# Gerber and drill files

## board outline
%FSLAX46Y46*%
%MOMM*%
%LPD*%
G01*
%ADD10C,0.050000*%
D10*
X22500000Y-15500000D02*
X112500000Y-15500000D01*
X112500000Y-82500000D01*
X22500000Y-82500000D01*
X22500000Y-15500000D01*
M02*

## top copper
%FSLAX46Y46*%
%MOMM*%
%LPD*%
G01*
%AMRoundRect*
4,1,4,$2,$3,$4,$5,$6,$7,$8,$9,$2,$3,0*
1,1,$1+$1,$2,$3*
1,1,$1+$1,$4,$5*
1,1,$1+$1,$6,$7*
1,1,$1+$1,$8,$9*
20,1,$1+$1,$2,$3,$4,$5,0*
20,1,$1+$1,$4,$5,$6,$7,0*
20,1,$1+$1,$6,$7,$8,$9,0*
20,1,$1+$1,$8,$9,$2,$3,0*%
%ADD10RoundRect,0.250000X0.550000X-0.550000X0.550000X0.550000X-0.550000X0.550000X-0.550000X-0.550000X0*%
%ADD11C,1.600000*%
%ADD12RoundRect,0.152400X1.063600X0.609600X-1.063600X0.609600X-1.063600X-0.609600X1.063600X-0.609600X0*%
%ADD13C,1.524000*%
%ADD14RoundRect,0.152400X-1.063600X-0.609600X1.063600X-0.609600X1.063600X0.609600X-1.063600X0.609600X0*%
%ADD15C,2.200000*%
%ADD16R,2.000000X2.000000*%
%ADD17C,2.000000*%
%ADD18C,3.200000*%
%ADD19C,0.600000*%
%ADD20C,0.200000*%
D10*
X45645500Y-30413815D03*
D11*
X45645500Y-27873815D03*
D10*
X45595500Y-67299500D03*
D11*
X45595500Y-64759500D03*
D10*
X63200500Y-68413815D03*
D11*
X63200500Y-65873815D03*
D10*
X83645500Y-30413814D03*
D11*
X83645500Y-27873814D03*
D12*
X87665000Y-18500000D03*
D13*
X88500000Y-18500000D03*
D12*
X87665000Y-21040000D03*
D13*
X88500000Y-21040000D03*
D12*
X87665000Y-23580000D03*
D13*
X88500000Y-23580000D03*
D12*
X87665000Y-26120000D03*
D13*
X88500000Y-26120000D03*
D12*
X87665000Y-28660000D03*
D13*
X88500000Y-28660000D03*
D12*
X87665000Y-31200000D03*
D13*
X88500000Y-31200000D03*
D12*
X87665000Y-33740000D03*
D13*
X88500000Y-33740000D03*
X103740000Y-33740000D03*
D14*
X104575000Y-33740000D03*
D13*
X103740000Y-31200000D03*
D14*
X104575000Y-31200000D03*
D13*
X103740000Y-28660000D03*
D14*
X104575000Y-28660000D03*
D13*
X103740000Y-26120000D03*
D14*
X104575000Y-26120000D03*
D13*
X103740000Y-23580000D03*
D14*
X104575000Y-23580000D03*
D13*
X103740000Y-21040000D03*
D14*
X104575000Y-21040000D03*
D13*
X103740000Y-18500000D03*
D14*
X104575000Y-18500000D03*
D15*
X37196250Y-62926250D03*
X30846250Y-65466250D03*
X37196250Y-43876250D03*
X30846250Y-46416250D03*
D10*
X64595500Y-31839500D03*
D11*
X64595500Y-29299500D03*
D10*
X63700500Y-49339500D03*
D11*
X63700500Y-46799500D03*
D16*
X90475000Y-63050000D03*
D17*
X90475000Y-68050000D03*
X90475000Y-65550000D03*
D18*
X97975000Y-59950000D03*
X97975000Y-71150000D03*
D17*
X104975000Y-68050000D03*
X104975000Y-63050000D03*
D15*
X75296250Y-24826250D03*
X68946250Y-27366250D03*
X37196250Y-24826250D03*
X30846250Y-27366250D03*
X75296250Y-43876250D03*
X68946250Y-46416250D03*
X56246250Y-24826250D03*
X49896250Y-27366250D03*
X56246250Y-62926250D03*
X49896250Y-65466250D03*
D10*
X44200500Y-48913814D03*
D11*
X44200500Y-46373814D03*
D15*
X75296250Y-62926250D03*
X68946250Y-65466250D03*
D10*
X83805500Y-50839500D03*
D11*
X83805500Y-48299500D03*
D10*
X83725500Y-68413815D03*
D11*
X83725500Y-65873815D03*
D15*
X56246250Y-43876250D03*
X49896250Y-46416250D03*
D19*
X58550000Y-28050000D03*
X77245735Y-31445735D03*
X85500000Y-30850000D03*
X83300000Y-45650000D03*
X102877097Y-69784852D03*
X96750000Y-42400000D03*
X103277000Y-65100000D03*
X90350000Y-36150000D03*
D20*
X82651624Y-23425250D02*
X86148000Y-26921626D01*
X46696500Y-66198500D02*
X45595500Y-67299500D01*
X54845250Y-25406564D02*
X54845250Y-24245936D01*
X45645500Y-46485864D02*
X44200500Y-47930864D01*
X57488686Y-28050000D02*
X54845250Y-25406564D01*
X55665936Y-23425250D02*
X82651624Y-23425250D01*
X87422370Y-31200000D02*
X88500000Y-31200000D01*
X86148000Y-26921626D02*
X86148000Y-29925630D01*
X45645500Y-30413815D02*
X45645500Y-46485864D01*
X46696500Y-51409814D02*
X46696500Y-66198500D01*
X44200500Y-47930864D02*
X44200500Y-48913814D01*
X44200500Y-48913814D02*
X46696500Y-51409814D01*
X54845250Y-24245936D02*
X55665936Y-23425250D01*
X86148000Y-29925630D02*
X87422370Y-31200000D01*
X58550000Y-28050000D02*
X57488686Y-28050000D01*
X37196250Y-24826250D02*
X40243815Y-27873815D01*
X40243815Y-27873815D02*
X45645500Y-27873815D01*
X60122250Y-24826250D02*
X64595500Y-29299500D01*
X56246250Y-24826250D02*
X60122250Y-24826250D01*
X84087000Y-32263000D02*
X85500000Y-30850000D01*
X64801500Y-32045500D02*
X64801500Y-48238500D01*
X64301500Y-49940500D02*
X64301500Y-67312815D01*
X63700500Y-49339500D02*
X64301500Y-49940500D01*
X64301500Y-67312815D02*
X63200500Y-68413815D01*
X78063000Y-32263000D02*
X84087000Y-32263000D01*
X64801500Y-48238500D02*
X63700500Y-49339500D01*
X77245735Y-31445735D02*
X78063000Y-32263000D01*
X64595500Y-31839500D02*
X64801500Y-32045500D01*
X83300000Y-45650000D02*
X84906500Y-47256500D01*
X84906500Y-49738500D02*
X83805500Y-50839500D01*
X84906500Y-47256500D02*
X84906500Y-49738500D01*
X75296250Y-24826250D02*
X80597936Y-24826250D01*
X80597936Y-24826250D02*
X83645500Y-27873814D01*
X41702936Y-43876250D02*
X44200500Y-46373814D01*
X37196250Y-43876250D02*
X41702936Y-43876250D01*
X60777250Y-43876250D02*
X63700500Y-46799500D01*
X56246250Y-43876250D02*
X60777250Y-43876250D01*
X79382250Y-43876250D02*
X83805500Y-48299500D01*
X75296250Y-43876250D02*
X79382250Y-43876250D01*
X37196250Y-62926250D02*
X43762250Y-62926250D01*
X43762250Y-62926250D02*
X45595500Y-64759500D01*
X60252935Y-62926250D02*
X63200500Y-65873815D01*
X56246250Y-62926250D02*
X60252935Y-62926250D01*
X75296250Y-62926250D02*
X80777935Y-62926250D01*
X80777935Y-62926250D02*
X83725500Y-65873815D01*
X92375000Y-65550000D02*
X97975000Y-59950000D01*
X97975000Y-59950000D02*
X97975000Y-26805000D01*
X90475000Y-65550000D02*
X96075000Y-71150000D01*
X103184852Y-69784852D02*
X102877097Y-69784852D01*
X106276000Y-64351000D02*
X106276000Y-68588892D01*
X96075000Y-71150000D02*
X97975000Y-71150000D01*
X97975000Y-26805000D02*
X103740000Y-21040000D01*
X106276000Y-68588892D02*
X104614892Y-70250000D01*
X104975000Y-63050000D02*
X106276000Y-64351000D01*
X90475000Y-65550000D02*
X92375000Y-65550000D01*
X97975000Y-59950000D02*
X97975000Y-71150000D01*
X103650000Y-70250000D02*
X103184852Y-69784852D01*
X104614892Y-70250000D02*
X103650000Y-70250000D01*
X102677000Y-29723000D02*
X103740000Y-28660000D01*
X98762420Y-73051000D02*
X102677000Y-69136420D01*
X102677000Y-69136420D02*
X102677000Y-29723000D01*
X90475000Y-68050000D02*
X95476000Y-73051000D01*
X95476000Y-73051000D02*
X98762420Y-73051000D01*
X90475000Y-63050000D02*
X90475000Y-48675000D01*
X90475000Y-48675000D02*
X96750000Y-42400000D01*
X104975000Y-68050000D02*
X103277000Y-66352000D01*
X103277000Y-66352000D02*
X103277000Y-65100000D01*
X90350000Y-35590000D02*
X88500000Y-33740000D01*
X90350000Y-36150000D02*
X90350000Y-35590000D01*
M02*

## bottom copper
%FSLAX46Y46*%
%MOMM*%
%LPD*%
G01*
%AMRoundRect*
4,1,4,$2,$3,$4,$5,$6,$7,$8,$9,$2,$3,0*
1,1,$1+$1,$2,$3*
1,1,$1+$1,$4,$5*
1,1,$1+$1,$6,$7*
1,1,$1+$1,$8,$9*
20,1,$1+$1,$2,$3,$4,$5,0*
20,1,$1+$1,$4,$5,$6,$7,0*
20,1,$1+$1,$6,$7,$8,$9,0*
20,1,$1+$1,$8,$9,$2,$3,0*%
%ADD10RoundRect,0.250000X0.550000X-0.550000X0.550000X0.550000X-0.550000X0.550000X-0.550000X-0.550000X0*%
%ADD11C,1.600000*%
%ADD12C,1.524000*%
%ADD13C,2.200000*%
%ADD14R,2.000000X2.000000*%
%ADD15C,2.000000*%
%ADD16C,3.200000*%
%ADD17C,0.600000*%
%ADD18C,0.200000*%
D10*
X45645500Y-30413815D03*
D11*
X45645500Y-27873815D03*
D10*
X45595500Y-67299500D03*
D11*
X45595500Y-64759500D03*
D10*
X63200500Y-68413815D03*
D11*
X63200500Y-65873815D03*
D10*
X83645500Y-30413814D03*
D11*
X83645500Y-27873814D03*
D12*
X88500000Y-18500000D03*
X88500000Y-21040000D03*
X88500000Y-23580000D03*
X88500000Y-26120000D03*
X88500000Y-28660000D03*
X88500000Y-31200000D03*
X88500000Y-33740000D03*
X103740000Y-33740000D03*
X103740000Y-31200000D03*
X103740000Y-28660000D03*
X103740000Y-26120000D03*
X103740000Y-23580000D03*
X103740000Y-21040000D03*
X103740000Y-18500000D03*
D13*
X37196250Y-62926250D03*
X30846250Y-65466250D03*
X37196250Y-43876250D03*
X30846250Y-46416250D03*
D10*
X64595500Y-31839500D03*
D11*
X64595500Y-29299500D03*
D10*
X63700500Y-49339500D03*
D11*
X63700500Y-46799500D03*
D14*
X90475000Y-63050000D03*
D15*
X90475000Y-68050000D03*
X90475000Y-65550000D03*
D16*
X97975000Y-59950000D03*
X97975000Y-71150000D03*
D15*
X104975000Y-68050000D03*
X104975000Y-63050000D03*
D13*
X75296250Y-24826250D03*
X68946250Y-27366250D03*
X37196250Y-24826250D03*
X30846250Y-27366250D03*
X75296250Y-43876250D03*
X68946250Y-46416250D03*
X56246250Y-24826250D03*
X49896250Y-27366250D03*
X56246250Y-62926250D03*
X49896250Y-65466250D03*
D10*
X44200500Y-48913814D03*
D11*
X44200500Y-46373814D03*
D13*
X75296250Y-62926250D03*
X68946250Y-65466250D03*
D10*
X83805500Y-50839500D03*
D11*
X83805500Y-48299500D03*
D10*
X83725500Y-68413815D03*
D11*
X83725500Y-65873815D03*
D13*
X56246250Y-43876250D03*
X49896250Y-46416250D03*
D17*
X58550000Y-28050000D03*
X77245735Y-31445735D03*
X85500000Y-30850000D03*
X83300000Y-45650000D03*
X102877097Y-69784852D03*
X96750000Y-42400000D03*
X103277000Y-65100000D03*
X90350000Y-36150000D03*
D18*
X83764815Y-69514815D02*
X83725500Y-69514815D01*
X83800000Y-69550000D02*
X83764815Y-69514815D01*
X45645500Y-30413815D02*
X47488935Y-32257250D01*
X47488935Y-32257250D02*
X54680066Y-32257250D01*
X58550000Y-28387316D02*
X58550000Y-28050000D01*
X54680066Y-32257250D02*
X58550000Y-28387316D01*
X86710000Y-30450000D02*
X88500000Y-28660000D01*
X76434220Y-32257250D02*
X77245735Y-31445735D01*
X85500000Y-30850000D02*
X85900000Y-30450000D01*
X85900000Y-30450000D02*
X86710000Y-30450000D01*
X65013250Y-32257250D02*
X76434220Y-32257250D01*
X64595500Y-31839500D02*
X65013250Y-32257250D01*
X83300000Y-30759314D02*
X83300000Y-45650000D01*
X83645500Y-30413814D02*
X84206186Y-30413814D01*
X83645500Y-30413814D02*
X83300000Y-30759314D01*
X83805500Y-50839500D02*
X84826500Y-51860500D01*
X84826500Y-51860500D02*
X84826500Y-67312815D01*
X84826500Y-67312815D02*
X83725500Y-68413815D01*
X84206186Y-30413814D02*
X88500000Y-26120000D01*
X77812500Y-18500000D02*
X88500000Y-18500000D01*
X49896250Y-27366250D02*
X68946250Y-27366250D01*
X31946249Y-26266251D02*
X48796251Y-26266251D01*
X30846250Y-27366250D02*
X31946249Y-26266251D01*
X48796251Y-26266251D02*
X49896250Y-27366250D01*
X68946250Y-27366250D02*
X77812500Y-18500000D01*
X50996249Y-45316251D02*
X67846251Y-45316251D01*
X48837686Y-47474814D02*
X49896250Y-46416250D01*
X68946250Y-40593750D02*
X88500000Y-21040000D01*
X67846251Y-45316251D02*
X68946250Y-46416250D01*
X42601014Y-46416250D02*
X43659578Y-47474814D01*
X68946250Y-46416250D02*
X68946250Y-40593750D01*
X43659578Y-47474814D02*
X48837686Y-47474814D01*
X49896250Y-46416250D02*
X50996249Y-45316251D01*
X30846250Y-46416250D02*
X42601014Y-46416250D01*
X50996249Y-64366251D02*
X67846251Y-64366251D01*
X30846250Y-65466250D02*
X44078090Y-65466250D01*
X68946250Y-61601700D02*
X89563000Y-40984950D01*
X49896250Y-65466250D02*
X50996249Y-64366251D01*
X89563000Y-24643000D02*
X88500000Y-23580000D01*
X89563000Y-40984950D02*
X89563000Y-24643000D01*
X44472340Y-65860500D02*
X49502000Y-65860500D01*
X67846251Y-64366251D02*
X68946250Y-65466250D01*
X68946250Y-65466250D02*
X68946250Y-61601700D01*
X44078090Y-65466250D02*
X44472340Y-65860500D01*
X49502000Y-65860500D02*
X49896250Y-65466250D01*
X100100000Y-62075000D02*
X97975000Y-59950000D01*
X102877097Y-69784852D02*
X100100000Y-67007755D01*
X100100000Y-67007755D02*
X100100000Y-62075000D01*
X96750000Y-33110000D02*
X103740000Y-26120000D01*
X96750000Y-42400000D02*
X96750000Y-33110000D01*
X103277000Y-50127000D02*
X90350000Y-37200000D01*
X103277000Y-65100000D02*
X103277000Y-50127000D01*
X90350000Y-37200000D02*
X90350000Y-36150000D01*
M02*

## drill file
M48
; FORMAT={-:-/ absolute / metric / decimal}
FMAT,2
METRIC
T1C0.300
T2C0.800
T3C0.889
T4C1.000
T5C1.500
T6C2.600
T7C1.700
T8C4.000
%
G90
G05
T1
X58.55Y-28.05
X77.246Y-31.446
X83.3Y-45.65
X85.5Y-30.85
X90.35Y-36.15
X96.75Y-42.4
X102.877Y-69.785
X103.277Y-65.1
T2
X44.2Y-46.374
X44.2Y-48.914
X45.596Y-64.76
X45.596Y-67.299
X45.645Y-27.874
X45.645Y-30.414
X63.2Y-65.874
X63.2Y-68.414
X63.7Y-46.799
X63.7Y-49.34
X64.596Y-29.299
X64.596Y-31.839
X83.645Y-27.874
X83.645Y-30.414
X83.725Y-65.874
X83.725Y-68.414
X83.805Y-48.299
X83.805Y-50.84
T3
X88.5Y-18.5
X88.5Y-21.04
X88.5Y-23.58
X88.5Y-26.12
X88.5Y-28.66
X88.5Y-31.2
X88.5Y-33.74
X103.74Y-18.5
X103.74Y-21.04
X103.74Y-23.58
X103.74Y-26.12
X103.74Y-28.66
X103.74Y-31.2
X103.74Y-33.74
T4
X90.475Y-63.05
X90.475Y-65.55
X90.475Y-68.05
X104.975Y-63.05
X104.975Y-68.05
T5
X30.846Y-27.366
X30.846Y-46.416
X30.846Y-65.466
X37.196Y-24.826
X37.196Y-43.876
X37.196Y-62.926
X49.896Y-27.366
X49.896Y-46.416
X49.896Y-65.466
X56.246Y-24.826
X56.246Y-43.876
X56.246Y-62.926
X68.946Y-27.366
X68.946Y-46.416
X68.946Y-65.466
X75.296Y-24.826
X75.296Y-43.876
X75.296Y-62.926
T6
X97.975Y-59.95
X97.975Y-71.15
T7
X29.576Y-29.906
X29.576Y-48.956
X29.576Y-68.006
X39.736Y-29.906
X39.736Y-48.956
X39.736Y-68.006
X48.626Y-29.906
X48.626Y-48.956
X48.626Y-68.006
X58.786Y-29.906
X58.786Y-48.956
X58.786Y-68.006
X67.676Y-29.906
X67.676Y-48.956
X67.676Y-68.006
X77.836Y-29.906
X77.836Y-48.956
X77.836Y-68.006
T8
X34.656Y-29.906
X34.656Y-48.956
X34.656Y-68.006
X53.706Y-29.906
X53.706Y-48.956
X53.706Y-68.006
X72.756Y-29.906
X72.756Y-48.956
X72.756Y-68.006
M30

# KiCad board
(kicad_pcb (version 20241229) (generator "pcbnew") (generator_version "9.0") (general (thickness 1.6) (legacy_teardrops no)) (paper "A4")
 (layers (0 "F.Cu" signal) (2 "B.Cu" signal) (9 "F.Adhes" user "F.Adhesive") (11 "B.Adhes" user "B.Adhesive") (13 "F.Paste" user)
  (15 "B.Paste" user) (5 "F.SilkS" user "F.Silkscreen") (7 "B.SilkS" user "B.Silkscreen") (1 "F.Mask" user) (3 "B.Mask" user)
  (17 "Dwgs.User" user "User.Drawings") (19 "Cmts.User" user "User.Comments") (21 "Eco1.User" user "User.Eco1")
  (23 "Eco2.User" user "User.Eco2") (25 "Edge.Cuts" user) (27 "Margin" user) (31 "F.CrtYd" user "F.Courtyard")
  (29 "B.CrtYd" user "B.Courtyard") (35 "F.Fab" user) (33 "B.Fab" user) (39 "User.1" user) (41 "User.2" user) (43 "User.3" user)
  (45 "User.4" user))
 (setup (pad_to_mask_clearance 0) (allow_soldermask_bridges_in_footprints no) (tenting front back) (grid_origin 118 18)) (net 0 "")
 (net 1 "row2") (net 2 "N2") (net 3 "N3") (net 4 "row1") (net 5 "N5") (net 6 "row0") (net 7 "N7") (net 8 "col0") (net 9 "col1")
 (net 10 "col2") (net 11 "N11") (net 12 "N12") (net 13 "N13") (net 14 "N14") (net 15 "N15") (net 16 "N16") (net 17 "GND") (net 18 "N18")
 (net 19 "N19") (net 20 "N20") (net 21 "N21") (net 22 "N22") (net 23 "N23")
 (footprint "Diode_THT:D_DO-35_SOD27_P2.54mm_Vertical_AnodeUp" (layer "F.Cu") (at 45.6455 30.413815 90)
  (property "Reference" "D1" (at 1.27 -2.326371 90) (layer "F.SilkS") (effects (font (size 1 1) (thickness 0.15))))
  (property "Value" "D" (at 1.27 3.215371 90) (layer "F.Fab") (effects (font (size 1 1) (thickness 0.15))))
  (pad "1" thru_hole roundrect (at 0 0 90) (size 1.6 1.6) (drill 0.8) (layers "*.Cu" "*.Mask") (remove_unused_layers no)
   (roundrect_rratio 0.15625) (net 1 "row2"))
  (pad "2" thru_hole circle (at 2.54 0 90) (size 1.6 1.6) (drill 0.8) (layers "*.Cu" "*.Mask") (remove_unused_layers no) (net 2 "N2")))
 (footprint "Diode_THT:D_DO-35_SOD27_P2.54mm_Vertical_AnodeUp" (layer "F.Cu") (at 45.5955 67.2995 90)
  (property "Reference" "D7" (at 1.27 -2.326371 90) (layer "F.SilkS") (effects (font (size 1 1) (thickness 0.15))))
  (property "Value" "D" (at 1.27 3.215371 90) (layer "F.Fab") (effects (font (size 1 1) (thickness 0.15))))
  (pad "1" thru_hole roundrect (at 0 0 90) (size 1.6 1.6) (drill 0.8) (layers "*.Cu" "*.Mask") (remove_unused_layers no)
   (roundrect_rratio 0.15625) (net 1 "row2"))
  (pad "2" thru_hole circle (at 2.54 0 90) (size 1.6 1.6) (drill 0.8) (layers "*.Cu" "*.Mask") (remove_unused_layers no) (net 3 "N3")))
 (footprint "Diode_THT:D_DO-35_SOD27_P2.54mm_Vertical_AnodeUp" (layer "F.Cu") (at 63.2005 68.413815 90)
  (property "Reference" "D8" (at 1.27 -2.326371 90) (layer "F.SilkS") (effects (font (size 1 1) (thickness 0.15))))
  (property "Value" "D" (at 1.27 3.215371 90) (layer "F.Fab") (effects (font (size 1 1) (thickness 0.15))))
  (pad "1" thru_hole roundrect (at 0 0 90) (size 1.6 1.6) (drill 0.8) (layers "*.Cu" "*.Mask") (remove_unused_layers no)
   (roundrect_rratio 0.15625) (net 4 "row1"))
  (pad "2" thru_hole circle (at 2.54 0 90) (size 1.6 1.6) (drill 0.8) (layers "*.Cu" "*.Mask") (remove_unused_layers no) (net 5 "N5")))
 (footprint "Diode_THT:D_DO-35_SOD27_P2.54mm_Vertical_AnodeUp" (layer "F.Cu") (at 83.6455 30.413814 90)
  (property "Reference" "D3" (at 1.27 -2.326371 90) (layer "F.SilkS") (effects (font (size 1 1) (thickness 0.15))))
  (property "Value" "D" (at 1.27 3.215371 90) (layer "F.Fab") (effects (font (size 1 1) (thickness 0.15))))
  (pad "1" thru_hole roundrect (at 0 0 90) (size 1.6 1.6) (drill 0.8) (layers "*.Cu" "*.Mask") (remove_unused_layers no)
   (roundrect_rratio 0.15625) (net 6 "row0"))
  (pad "2" thru_hole circle (at 2.54 0 90) (size 1.6 1.6) (drill 0.8) (layers "*.Cu" "*.Mask") (remove_unused_layers no) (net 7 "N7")))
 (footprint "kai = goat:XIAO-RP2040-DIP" (layer "F.Cu") (at 96.12 26.12)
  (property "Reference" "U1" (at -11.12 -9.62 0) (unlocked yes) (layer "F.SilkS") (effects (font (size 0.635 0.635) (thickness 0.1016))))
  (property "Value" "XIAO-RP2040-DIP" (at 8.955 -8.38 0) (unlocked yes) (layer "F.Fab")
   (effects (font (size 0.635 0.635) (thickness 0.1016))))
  (pad "1" smd roundrect (at -8.455 -7.62 180) (size 2.432 1.524) (layers "F.Cu" "F.Mask") (roundrect_rratio 0.1) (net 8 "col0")
   (thermal_bridge_angle 45))
  (pad "1" thru_hole circle (at -7.62 -7.62 180) (size 1.524 1.524) (drill 0.889) (layers "*.Cu" "*.Mask") (remove_unused_layers no)
   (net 8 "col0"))
  (pad "2" smd roundrect (at -8.455 -5.08 180) (size 2.432 1.524) (layers "F.Cu" "F.Mask") (roundrect_rratio 0.1) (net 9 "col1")
   (thermal_bridge_angle 45))
  (pad "2" thru_hole circle (at -7.62 -5.08 180) (size 1.524 1.524) (drill 0.889) (layers "*.Cu" "*.Mask") (remove_unused_layers no)
   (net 9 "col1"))
  (pad "3" smd roundrect (at -8.455 -2.54 180) (size 2.432 1.524) (layers "F.Cu" "F.Mask") (roundrect_rratio 0.1) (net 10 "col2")
   (thermal_bridge_angle 45))
  (pad "3" thru_hole circle (at -7.62 -2.54 180) (size 1.524 1.524) (drill 0.889) (layers "*.Cu" "*.Mask") (remove_unused_layers no)
   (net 10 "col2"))
  (pad "4" smd roundrect (at -8.455 0 180) (size 2.432 1.524) (layers "F.Cu" "F.Mask") (roundrect_rratio 0.1) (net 6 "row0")
   (thermal_bridge_angle 45))
  (pad "4" thru_hole circle (at -7.62 0 180) (size 1.524 1.524) (drill 0.889) (layers "*.Cu" "*.Mask") (remove_unused_layers no)
   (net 6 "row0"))
  (pad "5" smd roundrect (at -8.455 2.54 180) (size 2.432 1.524) (layers "F.Cu" "F.Mask") (roundrect_rratio 0.1) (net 4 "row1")
   (thermal_bridge_angle 45))
  (pad "5" thru_hole circle (at -7.62 2.54 180) (size 1.524 1.524) (drill 0.889) (layers "*.Cu" "*.Mask") (remove_unused_layers no)
   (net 4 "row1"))
  (pad "6" smd roundrect (at -8.455 5.08 180) (size 2.432 1.524) (layers "F.Cu" "F.Mask") (roundrect_rratio 0.1) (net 1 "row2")
   (thermal_bridge_angle 45))
  (pad "6" thru_hole circle (at -7.62 5.08 180) (size 1.524 1.524) (drill 0.889) (layers "*.Cu" "*.Mask") (remove_unused_layers no)
   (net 1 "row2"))
  (pad "7" smd roundrect (at -8.455 7.62 180) (size 2.432 1.524) (layers "F.Cu" "F.Mask") (roundrect_rratio 0.1) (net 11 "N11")
   (thermal_bridge_angle 45))
  (pad "7" thru_hole circle (at -7.62 7.62 180) (size 1.524 1.524) (drill 0.889) (layers "*.Cu" "*.Mask") (remove_unused_layers no)
   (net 11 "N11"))
  (pad "8" thru_hole circle (at 7.62 7.62) (size 1.524 1.524) (drill 0.889) (layers "*.Cu" "*.Mask") (remove_unused_layers no)
   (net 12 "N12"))
  (pad "8" smd roundrect (at 8.455 7.62) (size 2.432 1.524) (layers "F.Cu" "F.Mask") (roundrect_rratio 0.1) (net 12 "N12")
   (thermal_bridge_angle 45))
  (pad "9" thru_hole circle (at 7.62 5.08) (size 1.524 1.524) (drill 0.889) (layers "*.Cu" "*.Mask") (remove_unused_layers no)
   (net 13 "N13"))
  (pad "9" smd roundrect (at 8.455 5.08) (size 2.432 1.524) (layers "F.Cu" "F.Mask") (roundrect_rratio 0.1) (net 13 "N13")
   (thermal_bridge_angle 45))
  (pad "10" thru_hole circle (at 7.62 2.54) (size 1.524 1.524) (drill 0.889) (layers "*.Cu" "*.Mask") (remove_unused_layers no)
   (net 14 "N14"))
  (pad "10" smd roundrect (at 8.455 2.54) (size 2.432 1.524) (layers "F.Cu" "F.Mask") (roundrect_rratio 0.1) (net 14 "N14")
   (thermal_bridge_angle 45))
  (pad "11" thru_hole circle (at 7.62 0) (size 1.524 1.524) (drill 0.889) (layers "*.Cu" "*.Mask") (remove_unused_layers no) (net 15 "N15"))
  (pad "11" smd roundrect (at 8.455 0) (size 2.432 1.524) (layers "F.Cu" "F.Mask") (roundrect_rratio 0.1) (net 15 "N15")
   (thermal_bridge_angle 45))
  (pad "12" thru_hole circle (at 7.62 -2.54) (size 1.524 1.524) (drill 0.889) (layers "*.Cu" "*.Mask") (remove_unused_layers no)
   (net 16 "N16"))
  (pad "12" smd roundrect (at 8.455 -2.54) (size 2.432 1.524) (layers "F.Cu" "F.Mask") (roundrect_rratio 0.1) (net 16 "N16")
   (thermal_bridge_angle 45))
  (pad "13" thru_hole circle (at 7.62 -5.08) (size 1.524 1.524) (drill 0.889) (layers "*.Cu" "*.Mask") (remove_unused_layers no)
   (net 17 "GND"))
  (pad "13" smd roundrect (at 8.455 -5.08) (size 2.432 1.524) (layers "F.Cu" "F.Mask") (roundrect_rratio 0.1) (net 17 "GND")
   (thermal_bridge_angle 45))
  (pad "14" thru_hole circle (at 7.62 -7.62) (size 1.524 1.524) (drill 0.889) (layers "*.Cu" "*.Mask") (remove_unused_layers no)
   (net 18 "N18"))
  (pad "14" smd roundrect (at 8.455 -7.62) (size 2.432 1.524) (layers "F.Cu" "F.Mask") (roundrect_rratio 0.1) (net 18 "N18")
   (thermal_bridge_angle 45)))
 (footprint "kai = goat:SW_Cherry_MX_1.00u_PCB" (layer "F.Cu") (at 37.19625 62.92625)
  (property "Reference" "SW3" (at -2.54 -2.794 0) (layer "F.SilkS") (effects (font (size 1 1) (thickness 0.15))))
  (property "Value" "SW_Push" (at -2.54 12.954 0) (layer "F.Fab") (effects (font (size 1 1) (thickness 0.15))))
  (pad "" np_thru_hole circle (at -7.62 5.08) (size 1.7 1.7) (drill 1.7) (layers "*.Cu" "*.Mask"))
  (pad "" np_thru_hole circle (at -2.54 5.08) (size 4 4) (drill 4) (layers "*.Cu" "*.Mask"))
  (pad "" np_thru_hole circle (at 2.54 5.08) (size 1.7 1.7) (drill 1.7) (layers "*.Cu" "*.Mask"))
  (pad "1" thru_hole circle (at 0 0) (size 2.2 2.2) (drill 1.5) (layers "*.Cu" "*.Mask") (remove_unused_layers no) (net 3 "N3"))
  (pad "2" thru_hole circle (at -6.35 2.54) (size 2.2 2.2) (drill 1.5) (layers "*.Cu" "*.Mask") (remove_unused_layers no) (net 10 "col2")))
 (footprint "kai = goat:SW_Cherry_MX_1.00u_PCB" (layer "F.Cu") (at 37.19625 43.87625)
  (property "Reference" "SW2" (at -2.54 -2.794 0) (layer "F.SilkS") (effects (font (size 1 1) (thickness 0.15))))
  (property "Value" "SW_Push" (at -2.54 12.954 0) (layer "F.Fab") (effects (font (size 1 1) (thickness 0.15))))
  (pad "" np_thru_hole circle (at -7.62 5.08) (size 1.7 1.7) (drill 1.7) (layers "*.Cu" "*.Mask"))
  (pad "" np_thru_hole circle (at -2.54 5.08) (size 4 4) (drill 4) (layers "*.Cu" "*.Mask"))
  (pad "" np_thru_hole circle (at 2.54 5.08) (size 1.7 1.7) (drill 1.7) (layers "*.Cu" "*.Mask"))
  (pad "1" thru_hole circle (at 0 0) (size 2.2 2.2) (drill 1.5) (layers "*.Cu" "*.Mask") (remove_unused_layers no) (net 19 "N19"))
  (pad "2" thru_hole circle (at -6.35 2.54) (size 2.2 2.2) (drill 1.5) (layers "*.Cu" "*.Mask") (remove_unused_layers no) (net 9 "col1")))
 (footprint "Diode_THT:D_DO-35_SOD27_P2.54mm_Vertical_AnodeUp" (layer "F.Cu") (at 64.5955 31.8395 90)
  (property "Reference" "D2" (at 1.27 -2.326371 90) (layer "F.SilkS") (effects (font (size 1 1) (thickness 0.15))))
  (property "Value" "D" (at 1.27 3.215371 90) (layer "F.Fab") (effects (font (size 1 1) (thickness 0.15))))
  (pad "1" thru_hole roundrect (at 0 0 90) (size 1.6 1.6) (drill 0.8) (layers "*.Cu" "*.Mask") (remove_unused_layers no)
   (roundrect_rratio 0.15625) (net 4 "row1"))
  (pad "2" thru_hole circle (at 2.54 0 90) (size 1.6 1.6) (drill 0.8) (layers "*.Cu" "*.Mask") (remove_unused_layers no) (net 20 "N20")))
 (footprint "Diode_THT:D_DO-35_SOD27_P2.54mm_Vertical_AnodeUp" (layer "F.Cu") (at 63.7005 49.3395 90)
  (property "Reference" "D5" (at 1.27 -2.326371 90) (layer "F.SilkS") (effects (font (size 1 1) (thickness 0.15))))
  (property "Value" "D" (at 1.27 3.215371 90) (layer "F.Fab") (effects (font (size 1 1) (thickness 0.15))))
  (pad "1" thru_hole roundrect (at 0 0 90) (size 1.6 1.6) (drill 0.8) (layers "*.Cu" "*.Mask") (remove_unused_layers no)
   (roundrect_rratio 0.15625) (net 4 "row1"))
  (pad "2" thru_hole circle (at 2.54 0 90) (size 1.6 1.6) (drill 0.8) (layers "*.Cu" "*.Mask") (remove_unused_layers no) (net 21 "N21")))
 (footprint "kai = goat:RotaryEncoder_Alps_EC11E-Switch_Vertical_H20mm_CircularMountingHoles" (layer "F.Cu") (at 90.475 63.05)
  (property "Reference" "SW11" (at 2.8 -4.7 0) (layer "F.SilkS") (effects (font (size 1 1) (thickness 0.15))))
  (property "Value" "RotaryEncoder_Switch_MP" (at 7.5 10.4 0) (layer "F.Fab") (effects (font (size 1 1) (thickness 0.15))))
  (pad "A" thru_hole rect (at 0 0) (size 2 2) (drill 1) (layers "*.Cu" "*.Mask") (remove_unused_layers no) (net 15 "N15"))
  (pad "B" thru_hole circle (at 0 5) (size 2 2) (drill 1) (layers "*.Cu" "*.Mask") (remove_unused_layers no) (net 14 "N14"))
  (pad "C" thru_hole circle (at 0 2.5) (size 2 2) (drill 1) (layers "*.Cu" "*.Mask") (remove_unused_layers no) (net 17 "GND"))
  (pad "MP" thru_hole circle (at 7.5 -3.1) (size 3.2 3.2) (drill 2.6) (layers "*.Cu" "*.Mask") (remove_unused_layers no) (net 17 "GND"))
  (pad "MP" thru_hole circle (at 7.5 8.1) (size 3.2 3.2) (drill 2.6) (layers "*.Cu" "*.Mask") (remove_unused_layers no) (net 17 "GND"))
  (pad "S1" thru_hole circle (at 14.5 5) (size 2 2) (drill 1) (layers "*.Cu" "*.Mask") (remove_unused_layers no) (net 11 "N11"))
  (pad "S2" thru_hole circle (at 14.5 0) (size 2 2) (drill 1) (layers "*.Cu" "*.Mask") (remove_unused_layers no) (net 17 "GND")))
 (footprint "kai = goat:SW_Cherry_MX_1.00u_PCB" (layer "F.Cu") (at 75.29625 24.82625)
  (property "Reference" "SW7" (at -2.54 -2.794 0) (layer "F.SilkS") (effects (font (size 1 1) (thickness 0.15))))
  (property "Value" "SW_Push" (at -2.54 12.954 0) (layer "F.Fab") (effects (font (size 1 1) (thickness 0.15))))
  (pad "" np_thru_hole circle (at -7.62 5.08) (size 1.7 1.7) (drill 1.7) (layers "*.Cu" "*.Mask"))
  (pad "" np_thru_hole circle (at -2.54 5.08) (size 4 4) (drill 4) (layers "*.Cu" "*.Mask"))
  (pad "" np_thru_hole circle (at 2.54 5.08) (size 1.7 1.7) (drill 1.7) (layers "*.Cu" "*.Mask"))
  (pad "1" thru_hole circle (at 0 0) (size 2.2 2.2) (drill 1.5) (layers "*.Cu" "*.Mask") (remove_unused_layers no) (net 7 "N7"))
  (pad "2" thru_hole circle (at -6.35 2.54) (size 2.2 2.2) (drill 1.5) (layers "*.Cu" "*.Mask") (remove_unused_layers no) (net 8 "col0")))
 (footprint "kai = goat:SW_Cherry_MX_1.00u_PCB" (layer "F.Cu") (at 37.19625 24.82625)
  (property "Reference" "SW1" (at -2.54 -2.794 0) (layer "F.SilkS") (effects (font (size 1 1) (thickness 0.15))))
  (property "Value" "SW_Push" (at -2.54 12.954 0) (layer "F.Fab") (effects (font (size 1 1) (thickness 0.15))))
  (pad "" np_thru_hole circle (at -7.62 5.08) (size 1.7 1.7) (drill 1.7) (layers "*.Cu" "*.Mask"))
  (pad "" np_thru_hole circle (at -2.54 5.08) (size 4 4) (drill 4) (layers "*.Cu" "*.Mask"))
  (pad "" np_thru_hole circle (at 2.54 5.08) (size 1.7 1.7) (drill 1.7) (layers "*.Cu" "*.Mask"))
  (pad "1" thru_hole circle (at 0 0) (size 2.2 2.2) (drill 1.5) (layers "*.Cu" "*.Mask") (remove_unused_layers no) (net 2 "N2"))
  (pad "2" thru_hole circle (at -6.35 2.54) (size 2.2 2.2) (drill 1.5) (layers "*.Cu" "*.Mask") (remove_unused_layers no) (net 8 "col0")))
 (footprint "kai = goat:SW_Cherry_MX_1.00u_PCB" (layer "F.Cu") (at 75.29625 43.87625)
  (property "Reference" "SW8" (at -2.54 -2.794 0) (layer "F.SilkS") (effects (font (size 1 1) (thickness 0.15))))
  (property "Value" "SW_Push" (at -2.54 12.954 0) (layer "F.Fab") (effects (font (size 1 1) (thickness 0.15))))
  (pad "" np_thru_hole circle (at -7.62 5.08) (size 1.7 1.7) (drill 1.7) (layers "*.Cu" "*.Mask"))
  (pad "" np_thru_hole circle (at -2.54 5.08) (size 4 4) (drill 4) (layers "*.Cu" "*.Mask"))
  (pad "" np_thru_hole circle (at 2.54 5.08) (size 1.7 1.7) (drill 1.7) (layers "*.Cu" "*.Mask"))
  (pad "1" thru_hole circle (at 0 0) (size 2.2 2.2) (drill 1.5) (layers "*.Cu" "*.Mask") (remove_unused_layers no) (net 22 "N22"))
  (pad "2" thru_hole circle (at -6.35 2.54) (size 2.2 2.2) (drill 1.5) (layers "*.Cu" "*.Mask") (remove_unused_layers no) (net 9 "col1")))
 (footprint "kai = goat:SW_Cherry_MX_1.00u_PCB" (layer "F.Cu") (at 56.24625 24.82625)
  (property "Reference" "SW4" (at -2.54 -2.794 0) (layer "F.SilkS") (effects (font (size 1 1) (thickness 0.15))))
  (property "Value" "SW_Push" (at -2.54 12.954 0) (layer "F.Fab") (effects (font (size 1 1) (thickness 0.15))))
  (pad "" np_thru_hole circle (at -7.62 5.08) (size 1.7 1.7) (drill 1.7) (layers "*.Cu" "*.Mask"))
  (pad "" np_thru_hole circle (at -2.54 5.08) (size 4 4) (drill 4) (layers "*.Cu" "*.Mask"))
  (pad "" np_thru_hole circle (at 2.54 5.08) (size 1.7 1.7) (drill 1.7) (layers "*.Cu" "*.Mask"))
  (pad "1" thru_hole circle (at 0 0) (size 2.2 2.2) (drill 1.5) (layers "*.Cu" "*.Mask") (remove_unused_layers no) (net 20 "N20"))
  (pad "2" thru_hole circle (at -6.35 2.54) (size 2.2 2.2) (drill 1.5) (layers "*.Cu" "*.Mask") (remove_unused_layers no) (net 8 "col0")))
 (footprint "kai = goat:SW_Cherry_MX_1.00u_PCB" (layer "F.Cu") (at 56.24625 62.92625)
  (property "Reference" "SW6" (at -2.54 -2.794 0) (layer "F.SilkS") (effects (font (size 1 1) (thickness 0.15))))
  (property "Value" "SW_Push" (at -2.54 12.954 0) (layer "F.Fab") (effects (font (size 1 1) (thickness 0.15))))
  (pad "" np_thru_hole circle (at -7.62 5.08) (size 1.7 1.7) (drill 1.7) (layers "*.Cu" "*.Mask"))
  (pad "" np_thru_hole circle (at -2.54 5.08) (size 4 4) (drill 4) (layers "*.Cu" "*.Mask"))
  (pad "" np_thru_hole circle (at 2.54 5.08) (size 1.7 1.7) (drill 1.7) (layers "*.Cu" "*.Mask"))
  (pad "1" thru_hole circle (at 0 0) (size 2.2 2.2) (drill 1.5) (layers "*.Cu" "*.Mask") (remove_unused_layers no) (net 5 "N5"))
  (pad "2" thru_hole circle (at -6.35 2.54) (size 2.2 2.2) (drill 1.5) (layers "*.Cu" "*.Mask") (remove_unused_layers no) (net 10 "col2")))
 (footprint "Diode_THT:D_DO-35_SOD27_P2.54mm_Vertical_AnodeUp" (layer "F.Cu") (at 44.2005 48.913814 90)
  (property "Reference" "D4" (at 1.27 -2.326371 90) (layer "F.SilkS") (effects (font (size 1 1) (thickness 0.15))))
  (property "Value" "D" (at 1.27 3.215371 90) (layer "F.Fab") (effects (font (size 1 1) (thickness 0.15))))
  (pad "1" thru_hole roundrect (at 0 0 90) (size 1.6 1.6) (drill 0.8) (layers "*.Cu" "*.Mask") (remove_unused_layers no)
   (roundrect_rratio 0.15625) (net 1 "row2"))
  (pad "2" thru_hole circle (at 2.54 0 90) (size 1.6 1.6) (drill 0.8) (layers "*.Cu" "*.Mask") (remove_unused_layers no) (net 19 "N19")))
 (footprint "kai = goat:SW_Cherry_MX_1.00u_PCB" (layer "F.Cu") (at 75.29625 62.92625)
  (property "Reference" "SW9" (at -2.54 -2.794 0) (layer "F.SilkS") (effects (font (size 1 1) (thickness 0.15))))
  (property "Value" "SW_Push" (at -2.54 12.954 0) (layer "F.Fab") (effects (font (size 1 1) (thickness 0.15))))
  (pad "" np_thru_hole circle (at -7.62 5.08) (size 1.7 1.7) (drill 1.7) (layers "*.Cu" "*.Mask"))
  (pad "" np_thru_hole circle (at -2.54 5.08) (size 4 4) (drill 4) (layers "*.Cu" "*.Mask"))
  (pad "" np_thru_hole circle (at 2.54 5.08) (size 1.7 1.7) (drill 1.7) (layers "*.Cu" "*.Mask"))
  (pad "1" thru_hole circle (at 0 0) (size 2.2 2.2) (drill 1.5) (layers "*.Cu" "*.Mask") (remove_unused_layers no) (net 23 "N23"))
  (pad "2" thru_hole circle (at -6.35 2.54) (size 2.2 2.2) (drill 1.5) (layers "*.Cu" "*.Mask") (remove_unused_layers no) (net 10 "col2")))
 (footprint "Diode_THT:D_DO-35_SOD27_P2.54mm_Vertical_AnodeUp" (layer "F.Cu") (at 83.8055 50.8395 90)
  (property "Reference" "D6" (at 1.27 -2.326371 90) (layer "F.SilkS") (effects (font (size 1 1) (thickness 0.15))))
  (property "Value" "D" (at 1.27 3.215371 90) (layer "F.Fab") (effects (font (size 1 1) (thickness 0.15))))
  (pad "1" thru_hole roundrect (at 0 0 90) (size 1.6 1.6) (drill 0.8) (layers "*.Cu" "*.Mask") (remove_unused_layers no)
   (roundrect_rratio 0.15625) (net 6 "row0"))
  (pad "2" thru_hole circle (at 2.54 0 90) (size 1.6 1.6) (drill 0.8) (layers "*.Cu" "*.Mask") (remove_unused_layers no) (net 22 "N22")))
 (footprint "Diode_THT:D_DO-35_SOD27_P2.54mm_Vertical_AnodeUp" (layer "F.Cu") (at 83.7255 68.413815 90)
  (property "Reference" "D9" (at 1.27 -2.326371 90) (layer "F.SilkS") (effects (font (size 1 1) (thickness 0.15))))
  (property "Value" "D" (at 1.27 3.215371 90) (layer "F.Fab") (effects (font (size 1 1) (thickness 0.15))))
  (pad "1" thru_hole roundrect (at 0 0 90) (size 1.6 1.6) (drill 0.8) (layers "*.Cu" "*.Mask") (remove_unused_layers no)
   (roundrect_rratio 0.15625) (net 6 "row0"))
  (pad "2" thru_hole circle (at 2.54 0 90) (size 1.6 1.6) (drill 0.8) (layers "*.Cu" "*.Mask") (remove_unused_layers no) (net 23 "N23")))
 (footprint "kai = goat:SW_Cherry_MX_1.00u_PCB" (layer "F.Cu") (at 56.24625 43.87625)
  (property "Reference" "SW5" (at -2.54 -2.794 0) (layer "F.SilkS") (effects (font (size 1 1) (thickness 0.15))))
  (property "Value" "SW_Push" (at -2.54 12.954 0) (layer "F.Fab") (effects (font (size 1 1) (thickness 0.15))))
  (pad "" np_thru_hole circle (at -7.62 5.08) (size 1.7 1.7) (drill 1.7) (layers "*.Cu" "*.Mask"))
  (pad "" np_thru_hole circle (at -2.54 5.08) (size 4 4) (drill 4) (layers "*.Cu" "*.Mask"))
  (pad "" np_thru_hole circle (at 2.54 5.08) (size 1.7 1.7) (drill 1.7) (layers "*.Cu" "*.Mask"))
  (pad "1" thru_hole circle (at 0 0) (size 2.2 2.2) (drill 1.5) (layers "*.Cu" "*.Mask") (remove_unused_layers no) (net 21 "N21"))
  (pad "2" thru_hole circle (at -6.35 2.54) (size 2.2 2.2) (drill 1.5) (layers "*.Cu" "*.Mask") (remove_unused_layers no) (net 9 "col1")))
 (gr_rect (start 22.5 15.5) (end 112.5 82.5) (stroke (width 0.05) (type default)) (fill no) (layer "Edge.Cuts"))
 (segment (start 83.764815 69.514815) (end 83.7255 69.514815) (width 0.2) (layer "B.Cu") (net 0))
 (segment (start 83.8 69.55) (end 83.764815 69.514815) (width 0.2) (layer "B.Cu") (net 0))
 (segment (start 82.651624 23.42525) (end 86.148 26.921626) (width 0.2) (layer "F.Cu") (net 1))
 (segment (start 46.6965 66.1985) (end 45.5955 67.2995) (width 0.2) (layer "F.Cu") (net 1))
 (segment (start 54.84525 25.406564) (end 54.84525 24.245936) (width 0.2) (layer "F.Cu") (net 1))
 (segment (start 45.6455 46.485864) (end 44.2005 47.930864) (width 0.2) (layer "F.Cu") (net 1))
 (segment (start 57.488686 28.05) (end 54.84525 25.406564) (width 0.2) (layer "F.Cu") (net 1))
 (segment (start 55.665936 23.42525) (end 82.651624 23.42525) (width 0.2) (layer "F.Cu") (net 1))
 (segment (start 87.42237 31.2) (end 88.5 31.2) (width 0.2) (layer "F.Cu") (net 1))
 (segment (start 86.148 26.921626) (end 86.148 29.92563) (width 0.2) (layer "F.Cu") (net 1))
 (segment (start 45.6455 30.413815) (end 45.6455 46.485864) (width 0.2) (layer "F.Cu") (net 1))
 (segment (start 46.6965 51.409814) (end 46.6965 66.1985) (width 0.2) (layer "F.Cu") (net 1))
 (segment (start 44.2005 47.930864) (end 44.2005 48.913814) (width 0.2) (layer "F.Cu") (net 1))
 (segment (start 44.2005 48.913814) (end 46.6965 51.409814) (width 0.2) (layer "F.Cu") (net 1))
 (segment (start 54.84525 24.245936) (end 55.665936 23.42525) (width 0.2) (layer "F.Cu") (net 1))
 (segment (start 86.148 29.92563) (end 87.42237 31.2) (width 0.2) (layer "F.Cu") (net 1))
 (segment (start 58.55 28.05) (end 57.488686 28.05) (width 0.2) (layer "F.Cu") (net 1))
 (via (at 58.55 28.05) (size 0.6) (drill 0.3) (layers "F.Cu" "B.Cu") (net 1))
 (segment (start 45.6455 30.413815) (end 47.488935 32.25725) (width 0.2) (layer "B.Cu") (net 1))
 (segment (start 47.488935 32.25725) (end 54.680066 32.25725) (width 0.2) (layer "B.Cu") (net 1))
 (segment (start 58.55 28.387316) (end 58.55 28.05) (width 0.2) (layer "B.Cu") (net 1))
 (segment (start 54.680066 32.25725) (end 58.55 28.387316) (width 0.2) (layer "B.Cu") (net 1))
 (segment (start 37.19625 24.82625) (end 40.243815 27.873815) (width 0.2) (layer "F.Cu") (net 2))
 (segment (start 40.243815 27.873815) (end 45.6455 27.873815) (width 0.2) (layer "F.Cu") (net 2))
 (segment (start 60.12225 24.82625) (end 64.5955 29.2995) (width 0.2) (layer "F.Cu") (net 20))
 (segment (start 56.24625 24.82625) (end 60.12225 24.82625) (width 0.2) (layer "F.Cu") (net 20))
 (segment (start 84.087 32.263) (end 85.5 30.85) (width 0.2) (layer "F.Cu") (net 4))
 (segment (start 64.8015 32.0455) (end 64.8015 48.2385) (width 0.2) (layer "F.Cu") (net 4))
 (segment (start 64.3015 49.9405) (end 64.3015 67.312815) (width 0.2) (layer "F.Cu") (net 4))
 (segment (start 63.7005 49.3395) (end 64.3015 49.9405) (width 0.2) (layer "F.Cu") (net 4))
 (segment (start 64.3015 67.312815) (end 63.2005 68.413815) (width 0.2) (layer "F.Cu") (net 4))
 (segment (start 78.063 32.263) (end 84.087 32.263) (width 0.2) (layer "F.Cu") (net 4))
 (segment (start 64.8015 48.2385) (end 63.7005 49.3395) (width 0.2) (layer "F.Cu") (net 4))
 (segment (start 77.245735 31.445735) (end 78.063 32.263) (width 0.2) (layer "F.Cu") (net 4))
 (segment (start 64.5955 31.8395) (end 64.8015 32.0455) (width 0.2) (layer "F.Cu") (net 4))
 (via (at 77.245735 31.445735) (size 0.6) (drill 0.3) (layers "F.Cu" "B.Cu") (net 4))
 (via (at 85.5 30.85) (size 0.6) (drill 0.3) (layers "F.Cu" "B.Cu") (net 4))
 (segment (start 86.71 30.45) (end 88.5 28.66) (width 0.2) (layer "B.Cu") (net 4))
 (segment (start 76.43422 32.25725) (end 77.245735 31.445735) (width 0.2) (layer "B.Cu") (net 4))
 (segment (start 85.5 30.85) (end 85.9 30.45) (width 0.2) (layer "B.Cu") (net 4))
 (segment (start 85.9 30.45) (end 86.71 30.45) (width 0.2) (layer "B.Cu") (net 4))
 (segment (start 65.01325 32.25725) (end 76.43422 32.25725) (width 0.2) (layer "B.Cu") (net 4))
 (segment (start 64.5955 31.8395) (end 65.01325 32.25725) (width 0.2) (layer "B.Cu") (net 4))
 (segment (start 83.3 45.65) (end 84.9065 47.2565) (width 0.2) (layer "F.Cu") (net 6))
 (segment (start 84.9065 49.7385) (end 83.8055 50.8395) (width 0.2) (layer "F.Cu") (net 6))
 (segment (start 84.9065 47.2565) (end 84.9065 49.7385) (width 0.2) (layer "F.Cu") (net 6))
 (via (at 83.3 45.65) (size 0.6) (drill 0.3) (layers "F.Cu" "B.Cu") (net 6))
 (segment (start 83.3 30.759314) (end 83.3 45.65) (width 0.2) (layer "B.Cu") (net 6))
 (segment (start 83.6455 30.413814) (end 84.206186 30.413814) (width 0.2) (layer "B.Cu") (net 6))
 (segment (start 83.6455 30.413814) (end 83.3 30.759314) (width 0.2) (layer "B.Cu") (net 6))
 (segment (start 83.8055 50.8395) (end 84.8265 51.8605) (width 0.2) (layer "B.Cu") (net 6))
 (segment (start 84.8265 51.8605) (end 84.8265 67.312815) (width 0.2) (layer "B.Cu") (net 6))
 (segment (start 84.8265 67.312815) (end 83.7255 68.413815) (width 0.2) (layer "B.Cu") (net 6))
 (segment (start 84.206186 30.413814) (end 88.5 26.12) (width 0.2) (layer "B.Cu") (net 6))
 (segment (start 75.29625 24.82625) (end 80.597936 24.82625) (width 0.2) (layer "F.Cu") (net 7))
 (segment (start 80.597936 24.82625) (end 83.6455 27.873814) (width 0.2) (layer "F.Cu") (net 7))
 (segment (start 41.702936 43.87625) (end 44.2005 46.373814) (width 0.2) (layer "F.Cu") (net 19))
 (segment (start 37.19625 43.87625) (end 41.702936 43.87625) (width 0.2) (layer "F.Cu") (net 19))
 (segment (start 60.77725 43.87625) (end 63.7005 46.7995) (width 0.2) (layer "F.Cu") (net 21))
 (segment (start 56.24625 43.87625) (end 60.77725 43.87625) (width 0.2) (layer "F.Cu") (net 21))
 (segment (start 79.38225 43.87625) (end 83.8055 48.2995) (width 0.2) (layer "F.Cu") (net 22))
 (segment (start 75.29625 43.87625) (end 79.38225 43.87625) (width 0.2) (layer "F.Cu") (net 22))
 (segment (start 37.19625 62.92625) (end 43.76225 62.92625) (width 0.2) (layer "F.Cu") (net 3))
 (segment (start 43.76225 62.92625) (end 45.5955 64.7595) (width 0.2) (layer "F.Cu") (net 3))
 (segment (start 60.252935 62.92625) (end 63.2005 65.873815) (width 0.2) (layer "F.Cu") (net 5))
 (segment (start 56.24625 62.92625) (end 60.252935 62.92625) (width 0.2) (layer "F.Cu") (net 5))
 (segment (start 75.29625 62.92625) (end 80.777935 62.92625) (width 0.2) (layer "F.Cu") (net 23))
 (segment (start 80.777935 62.92625) (end 83.7255 65.873815) (width 0.2) (layer "F.Cu") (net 23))
 (segment (start 77.8125 18.5) (end 88.5 18.5) (width 0.2) (layer "B.Cu") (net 8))
 (segment (start 49.89625 27.36625) (end 68.94625 27.36625) (width 0.2) (layer "B.Cu") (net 8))
 (segment (start 31.946249 26.266251) (end 48.796251 26.266251) (width 0.2) (layer "B.Cu") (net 8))
 (segment (start 30.84625 27.36625) (end 31.946249 26.266251) (width 0.2) (layer "B.Cu") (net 8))
 (segment (start 48.796251 26.266251) (end 49.89625 27.36625) (width 0.2) (layer "B.Cu") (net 8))
 (segment (start 68.94625 27.36625) (end 77.8125 18.5) (width 0.2) (layer "B.Cu") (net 8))
 (segment (start 50.996249 45.316251) (end 67.846251 45.316251) (width 0.2) (layer "B.Cu") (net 9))
 (segment (start 48.837686 47.474814) (end 49.89625 46.41625) (width 0.2) (layer "B.Cu") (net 9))
 (segment (start 68.94625 40.59375) (end 88.5 21.04) (width 0.2) (layer "B.Cu") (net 9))
 (segment (start 67.846251 45.316251) (end 68.94625 46.41625) (width 0.2) (layer "B.Cu") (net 9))
 (segment (start 42.601014 46.41625) (end 43.659578 47.474814) (width 0.2) (layer "B.Cu") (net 9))
 (segment (start 68.94625 46.41625) (end 68.94625 40.59375) (width 0.2) (layer "B.Cu") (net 9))
 (segment (start 43.659578 47.474814) (end 48.837686 47.474814) (width 0.2) (layer "B.Cu") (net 9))
 (segment (start 49.89625 46.41625) (end 50.996249 45.316251) (width 0.2) (layer "B.Cu") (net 9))
 (segment (start 30.84625 46.41625) (end 42.601014 46.41625) (width 0.2) (layer "B.Cu") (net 9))
 (segment (start 50.996249 64.366251) (end 67.846251 64.366251) (width 0.2) (layer "B.Cu") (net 10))
 (segment (start 30.84625 65.46625) (end 44.07809 65.46625) (width 0.2) (layer "B.Cu") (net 10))
 (segment (start 68.94625 61.6017) (end 89.563 40.98495) (width 0.2) (layer "B.Cu") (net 10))
 (segment (start 49.89625 65.46625) (end 50.996249 64.366251) (width 0.2) (layer "B.Cu") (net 10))
 (segment (start 89.563 24.643) (end 88.5 23.58) (width 0.2) (layer "B.Cu") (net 10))
 (segment (start 89.563 40.98495) (end 89.563 24.643) (width 0.2) (layer "B.Cu") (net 10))
 (segment (start 44.47234 65.8605) (end 49.502 65.8605) (width 0.2) (layer "B.Cu") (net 10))
 (segment (start 67.846251 64.366251) (end 68.94625 65.46625) (width 0.2) (layer "B.Cu") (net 10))
 (segment (start 68.94625 65.46625) (end 68.94625 61.6017) (width 0.2) (layer "B.Cu") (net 10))
 (segment (start 44.07809 65.46625) (end 44.47234 65.8605) (width 0.2) (layer "B.Cu") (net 10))
 (segment (start 49.502 65.8605) (end 49.89625 65.46625) (width 0.2) (layer "B.Cu") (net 10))
 (segment (start 92.375 65.55) (end 97.975 59.95) (width 0.2) (layer "F.Cu") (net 17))
 (segment (start 97.975 59.95) (end 97.975 26.805) (width 0.2) (layer "F.Cu") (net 17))
 (segment (start 90.475 65.55) (end 96.075 71.15) (width 0.2) (layer "F.Cu") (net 17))
 (segment (start 103.184852 69.784852) (end 102.877097 69.784852) (width 0.2) (layer "F.Cu") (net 17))
 (segment (start 106.276 64.351) (end 106.276 68.588892) (width 0.2) (layer "F.Cu") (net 17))
 (segment (start 96.075 71.15) (end 97.975 71.15) (width 0.2) (layer "F.Cu") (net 17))
 (segment (start 97.975 26.805) (end 103.74 21.04) (width 0.2) (layer "F.Cu") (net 17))
 (segment (start 106.276 68.588892) (end 104.614892 70.25) (width 0.2) (layer "F.Cu") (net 17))
 (segment (start 104.975 63.05) (end 106.276 64.351) (width 0.2) (layer "F.Cu") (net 17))
 (segment (start 90.475 65.55) (end 92.375 65.55) (width 0.2) (layer "F.Cu") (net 17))
 (segment (start 97.975 59.95) (end 97.975 71.15) (width 0.2) (layer "F.Cu") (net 17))
 (segment (start 103.65 70.25) (end 103.184852 69.784852) (width 0.2) (layer "F.Cu") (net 17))
 (segment (start 104.614892 70.25) (end 103.65 70.25) (width 0.2) (layer "F.Cu") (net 17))
 (via (at 102.877097 69.784852) (size 0.6) (drill 0.3) (layers "F.Cu" "B.Cu") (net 17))
 (segment (start 100.1 62.075) (end 97.975 59.95) (width 0.2) (layer "B.Cu") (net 17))
 (segment (start 102.877097 69.784852) (end 100.1 67.007755) (width 0.2) (layer "B.Cu") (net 17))
 (segment (start 100.1 67.007755) (end 100.1 62.075) (width 0.2) (layer "B.Cu") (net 17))
 (segment (start 102.677 29.723) (end 103.74 28.66) (width 0.2) (layer "F.Cu") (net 14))
 (segment (start 98.76242 73.051) (end 102.677 69.13642) (width 0.2) (layer "F.Cu") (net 14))
 (segment (start 102.677 69.13642) (end 102.677 29.723) (width 0.2) (layer "F.Cu") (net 14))
 (segment (start 90.475 68.05) (end 95.476 73.051) (width 0.2) (layer "F.Cu") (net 14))
 (segment (start 95.476 73.051) (end 98.76242 73.051) (width 0.2) (layer "F.Cu") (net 14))
 (segment (start 90.475 63.05) (end 90.475 48.675) (width 0.2) (layer "F.Cu") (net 15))
 (segment (start 90.475 48.675) (end 96.75 42.4) (width 0.2) (layer "F.Cu") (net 15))
 (via (at 96.75 42.4) (size 0.6) (drill 0.3) (layers "F.Cu" "B.Cu") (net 15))
 (segment (start 96.75 33.11) (end 103.74 26.12) (width 0.2) (layer "B.Cu") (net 15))
 (segment (start 96.75 42.4) (end 96.75 33.11) (width 0.2) (layer "B.Cu") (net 15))
 (segment (start 104.975 68.05) (end 103.277 66.352) (width 0.2) (layer "F.Cu") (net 11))
 (segment (start 103.277 66.352) (end 103.277 65.1) (width 0.2) (layer "F.Cu") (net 11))
 (segment (start 90.35 35.59) (end 88.5 33.74) (width 0.2) (layer "F.Cu") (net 11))
 (segment (start 90.35 36.15) (end 90.35 35.59) (width 0.2) (layer "F.Cu") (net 11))
 (via (at 103.277 65.1) (size 0.6) (drill 0.3) (layers "F.Cu" "B.Cu") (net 11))
 (via (at 90.35 36.15) (size 0.6) (drill 0.3) (layers "F.Cu" "B.Cu") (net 11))
 (segment (start 103.277 50.127) (end 90.35 37.2) (width 0.2) (layer "B.Cu") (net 11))
 (segment (start 103.277 65.1) (end 103.277 50.127) (width 0.2) (layer "B.Cu") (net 11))
 (segment (start 90.35 37.2) (end 90.35 36.15) (width 0.2) (layer "B.Cu") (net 11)))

